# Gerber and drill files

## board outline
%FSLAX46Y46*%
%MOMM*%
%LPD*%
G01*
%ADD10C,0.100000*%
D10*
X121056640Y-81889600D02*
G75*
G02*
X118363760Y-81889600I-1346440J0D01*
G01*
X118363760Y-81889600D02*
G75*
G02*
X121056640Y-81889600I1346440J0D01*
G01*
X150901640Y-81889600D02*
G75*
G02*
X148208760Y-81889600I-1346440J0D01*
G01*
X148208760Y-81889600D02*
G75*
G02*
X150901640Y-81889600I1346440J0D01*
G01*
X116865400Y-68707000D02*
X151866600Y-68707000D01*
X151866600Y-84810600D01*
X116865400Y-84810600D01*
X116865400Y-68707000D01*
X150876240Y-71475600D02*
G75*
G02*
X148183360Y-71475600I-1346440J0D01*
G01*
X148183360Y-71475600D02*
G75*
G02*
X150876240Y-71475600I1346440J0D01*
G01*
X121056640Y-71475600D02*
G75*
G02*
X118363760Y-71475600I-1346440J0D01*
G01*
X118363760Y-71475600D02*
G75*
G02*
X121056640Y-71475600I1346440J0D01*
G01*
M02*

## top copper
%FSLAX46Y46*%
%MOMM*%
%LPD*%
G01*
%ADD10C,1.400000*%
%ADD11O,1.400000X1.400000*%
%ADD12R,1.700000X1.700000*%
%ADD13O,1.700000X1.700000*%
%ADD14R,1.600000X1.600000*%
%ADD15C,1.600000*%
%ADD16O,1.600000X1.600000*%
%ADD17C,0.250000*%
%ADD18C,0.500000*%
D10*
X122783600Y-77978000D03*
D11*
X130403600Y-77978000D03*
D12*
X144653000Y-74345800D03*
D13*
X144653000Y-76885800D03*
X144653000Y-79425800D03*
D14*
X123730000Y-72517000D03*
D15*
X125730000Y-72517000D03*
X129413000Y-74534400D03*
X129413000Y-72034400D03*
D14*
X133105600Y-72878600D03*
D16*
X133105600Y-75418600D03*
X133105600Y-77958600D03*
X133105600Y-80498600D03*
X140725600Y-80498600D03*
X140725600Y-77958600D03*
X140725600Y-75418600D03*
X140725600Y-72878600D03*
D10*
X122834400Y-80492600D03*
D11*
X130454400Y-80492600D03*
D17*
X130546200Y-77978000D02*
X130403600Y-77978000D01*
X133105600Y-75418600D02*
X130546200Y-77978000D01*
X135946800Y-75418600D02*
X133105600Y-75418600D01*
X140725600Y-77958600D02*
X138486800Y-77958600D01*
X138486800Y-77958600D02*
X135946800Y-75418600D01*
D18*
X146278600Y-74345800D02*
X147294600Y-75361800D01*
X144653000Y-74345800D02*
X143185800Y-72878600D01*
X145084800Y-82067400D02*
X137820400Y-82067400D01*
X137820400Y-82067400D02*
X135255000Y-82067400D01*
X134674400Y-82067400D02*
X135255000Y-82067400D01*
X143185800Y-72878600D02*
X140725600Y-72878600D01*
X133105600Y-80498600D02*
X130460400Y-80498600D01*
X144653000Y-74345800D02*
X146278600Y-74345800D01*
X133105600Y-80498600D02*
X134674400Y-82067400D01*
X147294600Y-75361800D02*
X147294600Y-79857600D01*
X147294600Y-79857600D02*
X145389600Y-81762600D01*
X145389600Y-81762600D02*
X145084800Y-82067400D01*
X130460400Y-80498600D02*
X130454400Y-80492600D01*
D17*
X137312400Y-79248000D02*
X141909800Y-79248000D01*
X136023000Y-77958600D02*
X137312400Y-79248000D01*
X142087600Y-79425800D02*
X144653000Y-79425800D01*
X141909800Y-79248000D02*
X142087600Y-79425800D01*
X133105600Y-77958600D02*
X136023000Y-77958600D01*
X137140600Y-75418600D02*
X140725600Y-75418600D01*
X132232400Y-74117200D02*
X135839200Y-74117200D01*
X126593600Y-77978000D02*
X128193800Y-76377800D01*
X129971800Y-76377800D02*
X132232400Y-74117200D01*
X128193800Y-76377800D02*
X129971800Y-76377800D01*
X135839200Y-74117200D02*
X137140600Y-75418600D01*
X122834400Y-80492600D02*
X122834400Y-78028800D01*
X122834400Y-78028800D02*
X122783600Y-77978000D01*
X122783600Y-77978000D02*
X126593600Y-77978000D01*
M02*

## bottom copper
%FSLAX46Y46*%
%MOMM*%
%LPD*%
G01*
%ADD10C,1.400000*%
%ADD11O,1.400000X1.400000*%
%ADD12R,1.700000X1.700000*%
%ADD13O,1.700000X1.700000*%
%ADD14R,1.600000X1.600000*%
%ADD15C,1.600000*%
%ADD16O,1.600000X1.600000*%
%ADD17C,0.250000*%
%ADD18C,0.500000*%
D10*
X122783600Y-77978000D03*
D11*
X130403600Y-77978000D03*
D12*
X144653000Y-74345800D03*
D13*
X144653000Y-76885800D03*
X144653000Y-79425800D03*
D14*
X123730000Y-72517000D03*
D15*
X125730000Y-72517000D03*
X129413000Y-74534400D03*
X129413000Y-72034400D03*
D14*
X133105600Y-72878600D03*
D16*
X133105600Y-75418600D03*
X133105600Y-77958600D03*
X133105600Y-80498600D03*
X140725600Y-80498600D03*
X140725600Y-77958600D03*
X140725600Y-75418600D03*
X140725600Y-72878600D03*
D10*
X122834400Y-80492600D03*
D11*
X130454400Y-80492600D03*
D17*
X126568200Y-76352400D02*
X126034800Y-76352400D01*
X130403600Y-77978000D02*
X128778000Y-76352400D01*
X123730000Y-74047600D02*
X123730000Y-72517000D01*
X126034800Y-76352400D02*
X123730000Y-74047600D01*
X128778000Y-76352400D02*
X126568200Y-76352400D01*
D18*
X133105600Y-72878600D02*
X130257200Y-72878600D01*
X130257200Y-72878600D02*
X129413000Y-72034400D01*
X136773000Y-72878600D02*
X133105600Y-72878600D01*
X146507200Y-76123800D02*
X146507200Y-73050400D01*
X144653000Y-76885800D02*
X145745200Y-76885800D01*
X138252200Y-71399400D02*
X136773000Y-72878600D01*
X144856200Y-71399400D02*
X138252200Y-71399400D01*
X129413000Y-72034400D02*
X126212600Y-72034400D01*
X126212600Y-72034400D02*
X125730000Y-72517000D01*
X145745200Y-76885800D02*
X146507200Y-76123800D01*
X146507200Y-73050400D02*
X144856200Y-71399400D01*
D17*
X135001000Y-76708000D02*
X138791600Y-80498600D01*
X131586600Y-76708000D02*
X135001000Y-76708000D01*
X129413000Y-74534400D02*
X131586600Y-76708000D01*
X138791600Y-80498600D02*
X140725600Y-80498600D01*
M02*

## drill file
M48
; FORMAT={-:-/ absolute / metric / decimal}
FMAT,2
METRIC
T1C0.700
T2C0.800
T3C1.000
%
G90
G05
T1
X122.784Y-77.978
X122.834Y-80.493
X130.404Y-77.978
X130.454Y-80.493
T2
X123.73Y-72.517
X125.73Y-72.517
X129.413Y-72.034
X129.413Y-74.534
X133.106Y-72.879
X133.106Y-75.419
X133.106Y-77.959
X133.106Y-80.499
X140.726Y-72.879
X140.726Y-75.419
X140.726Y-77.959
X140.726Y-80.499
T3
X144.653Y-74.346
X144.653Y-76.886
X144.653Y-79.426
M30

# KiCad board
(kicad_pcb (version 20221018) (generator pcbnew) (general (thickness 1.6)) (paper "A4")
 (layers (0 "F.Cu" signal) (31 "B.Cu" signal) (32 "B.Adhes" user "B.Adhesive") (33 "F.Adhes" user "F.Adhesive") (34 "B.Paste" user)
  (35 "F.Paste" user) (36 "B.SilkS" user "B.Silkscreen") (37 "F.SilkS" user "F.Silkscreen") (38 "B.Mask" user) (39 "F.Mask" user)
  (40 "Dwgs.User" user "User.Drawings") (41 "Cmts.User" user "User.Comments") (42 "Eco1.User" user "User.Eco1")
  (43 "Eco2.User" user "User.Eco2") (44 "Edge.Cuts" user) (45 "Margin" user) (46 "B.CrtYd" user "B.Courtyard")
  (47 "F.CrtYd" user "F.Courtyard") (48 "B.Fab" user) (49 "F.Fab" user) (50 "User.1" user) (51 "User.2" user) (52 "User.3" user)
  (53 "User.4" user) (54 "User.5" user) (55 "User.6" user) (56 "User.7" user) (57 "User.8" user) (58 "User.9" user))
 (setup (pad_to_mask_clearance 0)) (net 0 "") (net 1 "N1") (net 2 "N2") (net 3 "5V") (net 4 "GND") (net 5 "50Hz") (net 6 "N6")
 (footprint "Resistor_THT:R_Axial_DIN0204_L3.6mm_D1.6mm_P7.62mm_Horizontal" (layer "F.Cu") (at 122.7836 77.978)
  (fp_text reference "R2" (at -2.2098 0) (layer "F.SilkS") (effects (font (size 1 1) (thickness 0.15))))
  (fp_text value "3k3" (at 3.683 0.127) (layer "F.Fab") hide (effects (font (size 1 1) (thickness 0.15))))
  (pad "1" thru_hole circle (at 0 0) (size 1.4 1.4) (drill 0.7) (layers "*.Cu" "*.Mask") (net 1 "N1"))
  (pad "2" thru_hole oval (at 7.62 0) (size 1.4 1.4) (drill 0.7) (layers "*.Cu" "*.Mask") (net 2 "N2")))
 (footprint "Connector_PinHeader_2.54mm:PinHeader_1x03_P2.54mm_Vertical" (layer "F.Cu") (at 144.653 74.3458)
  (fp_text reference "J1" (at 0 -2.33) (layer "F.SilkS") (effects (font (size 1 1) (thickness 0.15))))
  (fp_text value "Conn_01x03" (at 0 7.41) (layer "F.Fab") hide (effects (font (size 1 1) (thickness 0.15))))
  (pad "1" thru_hole rect (at 0 0) (size 1.7 1.7) (drill 1) (layers "*.Cu" "*.Mask") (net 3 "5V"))
  (pad "2" thru_hole oval (at 0 2.54) (size 1.7 1.7) (drill 1) (layers "*.Cu" "*.Mask") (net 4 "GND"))
  (pad "3" thru_hole oval (at 0 5.08) (size 1.7 1.7) (drill 1) (layers "*.Cu" "*.Mask") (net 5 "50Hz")))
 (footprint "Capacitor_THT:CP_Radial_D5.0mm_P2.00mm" (layer "F.Cu") (at 123.73 72.517)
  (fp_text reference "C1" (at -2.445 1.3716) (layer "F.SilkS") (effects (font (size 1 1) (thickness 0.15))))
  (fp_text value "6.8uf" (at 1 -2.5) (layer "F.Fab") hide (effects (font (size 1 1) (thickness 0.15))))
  (pad "1" thru_hole rect (at 0 0) (size 1.6 1.6) (drill 0.8) (layers "*.Cu" "*.Mask") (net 2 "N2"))
  (pad "2" thru_hole circle (at 2 0) (size 1.6 1.6) (drill 0.8) (layers "*.Cu" "*.Mask") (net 4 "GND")))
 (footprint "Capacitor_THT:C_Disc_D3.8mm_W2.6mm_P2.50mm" (layer "F.Cu") (at 129.413 74.5344 90)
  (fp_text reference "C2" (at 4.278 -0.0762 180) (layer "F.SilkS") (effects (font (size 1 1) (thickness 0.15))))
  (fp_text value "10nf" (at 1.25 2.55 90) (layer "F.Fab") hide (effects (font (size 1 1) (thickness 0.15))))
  (pad "1" thru_hole circle (at 0 0 90) (size 1.6 1.6) (drill 0.8) (layers "*.Cu" "*.Mask") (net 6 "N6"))
  (pad "2" thru_hole circle (at 2.5 0 90) (size 1.6 1.6) (drill 0.8) (layers "*.Cu" "*.Mask") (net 4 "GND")))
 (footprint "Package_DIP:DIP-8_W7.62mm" (layer "F.Cu") (at 133.1056 72.8786)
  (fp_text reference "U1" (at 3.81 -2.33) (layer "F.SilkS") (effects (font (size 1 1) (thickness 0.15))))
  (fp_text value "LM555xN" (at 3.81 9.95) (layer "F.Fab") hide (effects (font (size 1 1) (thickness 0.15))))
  (pad "1" thru_hole rect (at 0 0) (size 1.6 1.6) (drill 0.8) (layers "*.Cu" "*.Mask") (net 4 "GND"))
  (pad "2" thru_hole oval (at 0 2.54) (size 1.6 1.6) (drill 0.8) (layers "*.Cu" "*.Mask") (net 2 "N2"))
  (pad "3" thru_hole oval (at 0 5.08) (size 1.6 1.6) (drill 0.8) (layers "*.Cu" "*.Mask") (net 5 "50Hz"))
  (pad "4" thru_hole oval (at 0 7.62) (size 1.6 1.6) (drill 0.8) (layers "*.Cu" "*.Mask") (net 3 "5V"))
  (pad "5" thru_hole oval (at 7.62 7.62) (size 1.6 1.6) (drill 0.8) (layers "*.Cu" "*.Mask") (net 6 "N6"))
  (pad "6" thru_hole oval (at 7.62 5.08) (size 1.6 1.6) (drill 0.8) (layers "*.Cu" "*.Mask") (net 2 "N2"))
  (pad "7" thru_hole oval (at 7.62 2.54) (size 1.6 1.6) (drill 0.8) (layers "*.Cu" "*.Mask") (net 1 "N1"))
  (pad "8" thru_hole oval (at 7.62 0) (size 1.6 1.6) (drill 0.8) (layers "*.Cu" "*.Mask") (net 3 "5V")))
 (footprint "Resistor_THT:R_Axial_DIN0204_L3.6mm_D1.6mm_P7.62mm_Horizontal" (layer "F.Cu") (at 122.8344 80.4926)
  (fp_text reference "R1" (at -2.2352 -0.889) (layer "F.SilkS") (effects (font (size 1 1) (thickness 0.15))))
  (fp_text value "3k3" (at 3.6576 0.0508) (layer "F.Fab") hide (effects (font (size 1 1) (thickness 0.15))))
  (pad "1" thru_hole circle (at 0 0) (size 1.4 1.4) (drill 0.7) (layers "*.Cu" "*.Mask") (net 1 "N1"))
  (pad "2" thru_hole oval (at 7.62 0) (size 1.4 1.4) (drill 0.7) (layers "*.Cu" "*.Mask") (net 3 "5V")))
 (gr_circle (center 119.7102 81.8896) (end 121.05664 81.8896) (stroke (width 0.1) (type default)) (fill none) (layer "Edge.Cuts"))
 (gr_circle (center 149.5552 81.8896) (end 150.9014 81.8642) (stroke (width 0.1) (type default)) (fill none) (layer "Edge.Cuts"))
 (gr_rect (start 116.8654 68.707) (end 151.8666 84.8106) (stroke (width 0.1) (type default)) (fill none) (layer "Edge.Cuts"))
 (gr_circle (center 149.5298 71.4756) (end 150.876 71.4502) (stroke (width 0.1) (type default)) (fill none) (layer "Edge.Cuts"))
 (gr_circle (center 119.7102 71.4756) (end 121.0564 71.4502) (stroke (width 0.1) (type default)) (fill none) (layer "Edge.Cuts"))
 (segment (start 130.5462 77.978) (end 130.4036 77.978) (width 0.25) (layer "F.Cu") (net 2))
 (segment (start 133.1056 75.4186) (end 130.5462 77.978) (width 0.25) (layer "F.Cu") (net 2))
 (segment (start 135.9468 75.4186) (end 133.1056 75.4186) (width 0.25) (layer "F.Cu") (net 2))
 (segment (start 140.7256 77.9586) (end 138.4868 77.9586) (width 0.25) (layer "F.Cu") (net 2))
 (segment (start 138.4868 77.9586) (end 135.9468 75.4186) (width 0.25) (layer "F.Cu") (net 2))
 (segment (start 126.5682 76.3524) (end 126.0348 76.3524) (width 0.25) (layer "B.Cu") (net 2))
 (segment (start 130.4036 77.978) (end 128.778 76.3524) (width 0.25) (layer "B.Cu") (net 2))
 (segment (start 123.73 74.0476) (end 123.73 72.517) (width 0.25) (layer "B.Cu") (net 2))
 (segment (start 126.0348 76.3524) (end 123.73 74.0476) (width 0.25) (layer "B.Cu") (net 2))
 (segment (start 128.778 76.3524) (end 126.5682 76.3524) (width 0.25) (layer "B.Cu") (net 2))
 (segment (start 133.1056 72.8786) (end 130.2572 72.8786) (width 0.5) (layer "B.Cu") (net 4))
 (segment (start 130.2572 72.8786) (end 129.413 72.0344) (width 0.5) (layer "B.Cu") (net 4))
 (segment (start 136.773 72.8786) (end 133.1056 72.8786) (width 0.5) (layer "B.Cu") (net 4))
 (segment (start 146.5072 76.1238) (end 146.5072 73.0504) (width 0.5) (layer "B.Cu") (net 4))
 (segment (start 144.653 76.8858) (end 145.7452 76.8858) (width 0.5) (layer "B.Cu") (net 4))
 (segment (start 138.2522 71.3994) (end 136.773 72.8786) (width 0.5) (layer "B.Cu") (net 4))
 (segment (start 144.8562 71.3994) (end 138.2522 71.3994) (width 0.5) (layer "B.Cu") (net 4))
 (segment (start 129.413 72.0344) (end 126.2126 72.0344) (width 0.5) (layer "B.Cu") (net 4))
 (segment (start 126.2126 72.0344) (end 125.73 72.517) (width 0.5) (layer "B.Cu") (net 4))
 (segment (start 145.7452 76.8858) (end 146.5072 76.1238) (width 0.5) (layer "B.Cu") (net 4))
 (segment (start 146.5072 73.0504) (end 144.8562 71.3994) (width 0.5) (layer "B.Cu") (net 4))
 (segment (start 135.001 76.708) (end 138.7916 80.4986) (width 0.25) (layer "B.Cu") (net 6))
 (segment (start 131.5866 76.708) (end 135.001 76.708) (width 0.25) (layer "B.Cu") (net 6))
 (segment (start 129.413 74.5344) (end 131.5866 76.708) (width 0.25) (layer "B.Cu") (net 6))
 (segment (start 138.7916 80.4986) (end 140.7256 80.4986) (width 0.25) (layer "B.Cu") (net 6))
 (segment (start 146.2786 74.3458) (end 147.2946 75.3618) (width 0.5) (layer "F.Cu") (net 3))
 (segment (start 144.653 74.3458) (end 143.1858 72.8786) (width 0.5) (layer "F.Cu") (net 3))
 (segment (start 145.0848 82.0674) (end 137.8204 82.0674) (width 0.5) (layer "F.Cu") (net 3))
 (segment (start 137.8204 82.0674) (end 135.255 82.0674) (width 0.5) (layer "F.Cu") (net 3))
 (segment (start 134.6744 82.0674) (end 135.255 82.0674) (width 0.5) (layer "F.Cu") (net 3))
 (segment (start 143.1858 72.8786) (end 140.7256 72.8786) (width 0.5) (layer "F.Cu") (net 3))
 (segment (start 133.1056 80.4986) (end 130.4604 80.4986) (width 0.5) (layer "F.Cu") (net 3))
 (segment (start 144.653 74.3458) (end 146.2786 74.3458) (width 0.5) (layer "F.Cu") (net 3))
 (segment (start 133.1056 80.4986) (end 134.6744 82.0674) (width 0.5) (layer "F.Cu") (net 3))
 (segment (start 147.2946 75.3618) (end 147.2946 79.8576) (width 0.5) (layer "F.Cu") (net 3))
 (segment (start 147.2946 79.8576) (end 145.3896 81.7626) (width 0.5) (layer "F.Cu") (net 3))
 (segment (start 145.3896 81.7626) (end 145.0848 82.0674) (width 0.5) (layer "F.Cu") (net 3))
 (segment (start 130.4604 80.4986) (end 130.4544 80.4926) (width 0.5) (layer "F.Cu") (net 3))
 (segment (start 137.3124 79.248) (end 141.9098 79.248) (width 0.25) (layer "F.Cu") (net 5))
 (segment (start 136.023 77.9586) (end 137.3124 79.248) (width 0.25) (layer "F.Cu") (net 5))
 (segment (start 142.0876 79.4258) (end 144.653 79.4258) (width 0.25) (layer "F.Cu") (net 5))
 (segment (start 141.9098 79.248) (end 142.0876 79.4258) (width 0.25) (layer "F.Cu") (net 5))
 (segment (start 133.1056 77.9586) (end 136.023 77.9586) (width 0.25) (layer "F.Cu") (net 5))
 (segment (start 137.1406 75.4186) (end 140.7256 75.4186) (width 0.25) (layer "F.Cu") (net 1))
 (segment (start 132.2324 74.1172) (end 135.8392 74.1172) (width 0.25) (layer "F.Cu") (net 1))
 (segment (start 126.5936 77.978) (end 128.1938 76.3778) (width 0.25) (layer "F.Cu") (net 1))
 (segment (start 129.9718 76.3778) (end 132.2324 74.1172) (width 0.25) (layer "F.Cu") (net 1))
 (segment (start 128.1938 76.3778) (end 129.9718 76.3778) (width 0.25) (layer "F.Cu") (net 1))
 (segment (start 135.8392 74.1172) (end 137.1406 75.4186) (width 0.25) (layer "F.Cu") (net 1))
 (segment (start 122.8344 80.4926) (end 122.8344 78.0288) (width 0.25) (layer "F.Cu") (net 1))
 (segment (start 122.8344 78.0288) (end 122.7836 77.978) (width 0.25) (layer "F.Cu") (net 1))
 (segment (start 122.7836 77.978) (end 126.5936 77.978) (width 0.25) (layer "F.Cu") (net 1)))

